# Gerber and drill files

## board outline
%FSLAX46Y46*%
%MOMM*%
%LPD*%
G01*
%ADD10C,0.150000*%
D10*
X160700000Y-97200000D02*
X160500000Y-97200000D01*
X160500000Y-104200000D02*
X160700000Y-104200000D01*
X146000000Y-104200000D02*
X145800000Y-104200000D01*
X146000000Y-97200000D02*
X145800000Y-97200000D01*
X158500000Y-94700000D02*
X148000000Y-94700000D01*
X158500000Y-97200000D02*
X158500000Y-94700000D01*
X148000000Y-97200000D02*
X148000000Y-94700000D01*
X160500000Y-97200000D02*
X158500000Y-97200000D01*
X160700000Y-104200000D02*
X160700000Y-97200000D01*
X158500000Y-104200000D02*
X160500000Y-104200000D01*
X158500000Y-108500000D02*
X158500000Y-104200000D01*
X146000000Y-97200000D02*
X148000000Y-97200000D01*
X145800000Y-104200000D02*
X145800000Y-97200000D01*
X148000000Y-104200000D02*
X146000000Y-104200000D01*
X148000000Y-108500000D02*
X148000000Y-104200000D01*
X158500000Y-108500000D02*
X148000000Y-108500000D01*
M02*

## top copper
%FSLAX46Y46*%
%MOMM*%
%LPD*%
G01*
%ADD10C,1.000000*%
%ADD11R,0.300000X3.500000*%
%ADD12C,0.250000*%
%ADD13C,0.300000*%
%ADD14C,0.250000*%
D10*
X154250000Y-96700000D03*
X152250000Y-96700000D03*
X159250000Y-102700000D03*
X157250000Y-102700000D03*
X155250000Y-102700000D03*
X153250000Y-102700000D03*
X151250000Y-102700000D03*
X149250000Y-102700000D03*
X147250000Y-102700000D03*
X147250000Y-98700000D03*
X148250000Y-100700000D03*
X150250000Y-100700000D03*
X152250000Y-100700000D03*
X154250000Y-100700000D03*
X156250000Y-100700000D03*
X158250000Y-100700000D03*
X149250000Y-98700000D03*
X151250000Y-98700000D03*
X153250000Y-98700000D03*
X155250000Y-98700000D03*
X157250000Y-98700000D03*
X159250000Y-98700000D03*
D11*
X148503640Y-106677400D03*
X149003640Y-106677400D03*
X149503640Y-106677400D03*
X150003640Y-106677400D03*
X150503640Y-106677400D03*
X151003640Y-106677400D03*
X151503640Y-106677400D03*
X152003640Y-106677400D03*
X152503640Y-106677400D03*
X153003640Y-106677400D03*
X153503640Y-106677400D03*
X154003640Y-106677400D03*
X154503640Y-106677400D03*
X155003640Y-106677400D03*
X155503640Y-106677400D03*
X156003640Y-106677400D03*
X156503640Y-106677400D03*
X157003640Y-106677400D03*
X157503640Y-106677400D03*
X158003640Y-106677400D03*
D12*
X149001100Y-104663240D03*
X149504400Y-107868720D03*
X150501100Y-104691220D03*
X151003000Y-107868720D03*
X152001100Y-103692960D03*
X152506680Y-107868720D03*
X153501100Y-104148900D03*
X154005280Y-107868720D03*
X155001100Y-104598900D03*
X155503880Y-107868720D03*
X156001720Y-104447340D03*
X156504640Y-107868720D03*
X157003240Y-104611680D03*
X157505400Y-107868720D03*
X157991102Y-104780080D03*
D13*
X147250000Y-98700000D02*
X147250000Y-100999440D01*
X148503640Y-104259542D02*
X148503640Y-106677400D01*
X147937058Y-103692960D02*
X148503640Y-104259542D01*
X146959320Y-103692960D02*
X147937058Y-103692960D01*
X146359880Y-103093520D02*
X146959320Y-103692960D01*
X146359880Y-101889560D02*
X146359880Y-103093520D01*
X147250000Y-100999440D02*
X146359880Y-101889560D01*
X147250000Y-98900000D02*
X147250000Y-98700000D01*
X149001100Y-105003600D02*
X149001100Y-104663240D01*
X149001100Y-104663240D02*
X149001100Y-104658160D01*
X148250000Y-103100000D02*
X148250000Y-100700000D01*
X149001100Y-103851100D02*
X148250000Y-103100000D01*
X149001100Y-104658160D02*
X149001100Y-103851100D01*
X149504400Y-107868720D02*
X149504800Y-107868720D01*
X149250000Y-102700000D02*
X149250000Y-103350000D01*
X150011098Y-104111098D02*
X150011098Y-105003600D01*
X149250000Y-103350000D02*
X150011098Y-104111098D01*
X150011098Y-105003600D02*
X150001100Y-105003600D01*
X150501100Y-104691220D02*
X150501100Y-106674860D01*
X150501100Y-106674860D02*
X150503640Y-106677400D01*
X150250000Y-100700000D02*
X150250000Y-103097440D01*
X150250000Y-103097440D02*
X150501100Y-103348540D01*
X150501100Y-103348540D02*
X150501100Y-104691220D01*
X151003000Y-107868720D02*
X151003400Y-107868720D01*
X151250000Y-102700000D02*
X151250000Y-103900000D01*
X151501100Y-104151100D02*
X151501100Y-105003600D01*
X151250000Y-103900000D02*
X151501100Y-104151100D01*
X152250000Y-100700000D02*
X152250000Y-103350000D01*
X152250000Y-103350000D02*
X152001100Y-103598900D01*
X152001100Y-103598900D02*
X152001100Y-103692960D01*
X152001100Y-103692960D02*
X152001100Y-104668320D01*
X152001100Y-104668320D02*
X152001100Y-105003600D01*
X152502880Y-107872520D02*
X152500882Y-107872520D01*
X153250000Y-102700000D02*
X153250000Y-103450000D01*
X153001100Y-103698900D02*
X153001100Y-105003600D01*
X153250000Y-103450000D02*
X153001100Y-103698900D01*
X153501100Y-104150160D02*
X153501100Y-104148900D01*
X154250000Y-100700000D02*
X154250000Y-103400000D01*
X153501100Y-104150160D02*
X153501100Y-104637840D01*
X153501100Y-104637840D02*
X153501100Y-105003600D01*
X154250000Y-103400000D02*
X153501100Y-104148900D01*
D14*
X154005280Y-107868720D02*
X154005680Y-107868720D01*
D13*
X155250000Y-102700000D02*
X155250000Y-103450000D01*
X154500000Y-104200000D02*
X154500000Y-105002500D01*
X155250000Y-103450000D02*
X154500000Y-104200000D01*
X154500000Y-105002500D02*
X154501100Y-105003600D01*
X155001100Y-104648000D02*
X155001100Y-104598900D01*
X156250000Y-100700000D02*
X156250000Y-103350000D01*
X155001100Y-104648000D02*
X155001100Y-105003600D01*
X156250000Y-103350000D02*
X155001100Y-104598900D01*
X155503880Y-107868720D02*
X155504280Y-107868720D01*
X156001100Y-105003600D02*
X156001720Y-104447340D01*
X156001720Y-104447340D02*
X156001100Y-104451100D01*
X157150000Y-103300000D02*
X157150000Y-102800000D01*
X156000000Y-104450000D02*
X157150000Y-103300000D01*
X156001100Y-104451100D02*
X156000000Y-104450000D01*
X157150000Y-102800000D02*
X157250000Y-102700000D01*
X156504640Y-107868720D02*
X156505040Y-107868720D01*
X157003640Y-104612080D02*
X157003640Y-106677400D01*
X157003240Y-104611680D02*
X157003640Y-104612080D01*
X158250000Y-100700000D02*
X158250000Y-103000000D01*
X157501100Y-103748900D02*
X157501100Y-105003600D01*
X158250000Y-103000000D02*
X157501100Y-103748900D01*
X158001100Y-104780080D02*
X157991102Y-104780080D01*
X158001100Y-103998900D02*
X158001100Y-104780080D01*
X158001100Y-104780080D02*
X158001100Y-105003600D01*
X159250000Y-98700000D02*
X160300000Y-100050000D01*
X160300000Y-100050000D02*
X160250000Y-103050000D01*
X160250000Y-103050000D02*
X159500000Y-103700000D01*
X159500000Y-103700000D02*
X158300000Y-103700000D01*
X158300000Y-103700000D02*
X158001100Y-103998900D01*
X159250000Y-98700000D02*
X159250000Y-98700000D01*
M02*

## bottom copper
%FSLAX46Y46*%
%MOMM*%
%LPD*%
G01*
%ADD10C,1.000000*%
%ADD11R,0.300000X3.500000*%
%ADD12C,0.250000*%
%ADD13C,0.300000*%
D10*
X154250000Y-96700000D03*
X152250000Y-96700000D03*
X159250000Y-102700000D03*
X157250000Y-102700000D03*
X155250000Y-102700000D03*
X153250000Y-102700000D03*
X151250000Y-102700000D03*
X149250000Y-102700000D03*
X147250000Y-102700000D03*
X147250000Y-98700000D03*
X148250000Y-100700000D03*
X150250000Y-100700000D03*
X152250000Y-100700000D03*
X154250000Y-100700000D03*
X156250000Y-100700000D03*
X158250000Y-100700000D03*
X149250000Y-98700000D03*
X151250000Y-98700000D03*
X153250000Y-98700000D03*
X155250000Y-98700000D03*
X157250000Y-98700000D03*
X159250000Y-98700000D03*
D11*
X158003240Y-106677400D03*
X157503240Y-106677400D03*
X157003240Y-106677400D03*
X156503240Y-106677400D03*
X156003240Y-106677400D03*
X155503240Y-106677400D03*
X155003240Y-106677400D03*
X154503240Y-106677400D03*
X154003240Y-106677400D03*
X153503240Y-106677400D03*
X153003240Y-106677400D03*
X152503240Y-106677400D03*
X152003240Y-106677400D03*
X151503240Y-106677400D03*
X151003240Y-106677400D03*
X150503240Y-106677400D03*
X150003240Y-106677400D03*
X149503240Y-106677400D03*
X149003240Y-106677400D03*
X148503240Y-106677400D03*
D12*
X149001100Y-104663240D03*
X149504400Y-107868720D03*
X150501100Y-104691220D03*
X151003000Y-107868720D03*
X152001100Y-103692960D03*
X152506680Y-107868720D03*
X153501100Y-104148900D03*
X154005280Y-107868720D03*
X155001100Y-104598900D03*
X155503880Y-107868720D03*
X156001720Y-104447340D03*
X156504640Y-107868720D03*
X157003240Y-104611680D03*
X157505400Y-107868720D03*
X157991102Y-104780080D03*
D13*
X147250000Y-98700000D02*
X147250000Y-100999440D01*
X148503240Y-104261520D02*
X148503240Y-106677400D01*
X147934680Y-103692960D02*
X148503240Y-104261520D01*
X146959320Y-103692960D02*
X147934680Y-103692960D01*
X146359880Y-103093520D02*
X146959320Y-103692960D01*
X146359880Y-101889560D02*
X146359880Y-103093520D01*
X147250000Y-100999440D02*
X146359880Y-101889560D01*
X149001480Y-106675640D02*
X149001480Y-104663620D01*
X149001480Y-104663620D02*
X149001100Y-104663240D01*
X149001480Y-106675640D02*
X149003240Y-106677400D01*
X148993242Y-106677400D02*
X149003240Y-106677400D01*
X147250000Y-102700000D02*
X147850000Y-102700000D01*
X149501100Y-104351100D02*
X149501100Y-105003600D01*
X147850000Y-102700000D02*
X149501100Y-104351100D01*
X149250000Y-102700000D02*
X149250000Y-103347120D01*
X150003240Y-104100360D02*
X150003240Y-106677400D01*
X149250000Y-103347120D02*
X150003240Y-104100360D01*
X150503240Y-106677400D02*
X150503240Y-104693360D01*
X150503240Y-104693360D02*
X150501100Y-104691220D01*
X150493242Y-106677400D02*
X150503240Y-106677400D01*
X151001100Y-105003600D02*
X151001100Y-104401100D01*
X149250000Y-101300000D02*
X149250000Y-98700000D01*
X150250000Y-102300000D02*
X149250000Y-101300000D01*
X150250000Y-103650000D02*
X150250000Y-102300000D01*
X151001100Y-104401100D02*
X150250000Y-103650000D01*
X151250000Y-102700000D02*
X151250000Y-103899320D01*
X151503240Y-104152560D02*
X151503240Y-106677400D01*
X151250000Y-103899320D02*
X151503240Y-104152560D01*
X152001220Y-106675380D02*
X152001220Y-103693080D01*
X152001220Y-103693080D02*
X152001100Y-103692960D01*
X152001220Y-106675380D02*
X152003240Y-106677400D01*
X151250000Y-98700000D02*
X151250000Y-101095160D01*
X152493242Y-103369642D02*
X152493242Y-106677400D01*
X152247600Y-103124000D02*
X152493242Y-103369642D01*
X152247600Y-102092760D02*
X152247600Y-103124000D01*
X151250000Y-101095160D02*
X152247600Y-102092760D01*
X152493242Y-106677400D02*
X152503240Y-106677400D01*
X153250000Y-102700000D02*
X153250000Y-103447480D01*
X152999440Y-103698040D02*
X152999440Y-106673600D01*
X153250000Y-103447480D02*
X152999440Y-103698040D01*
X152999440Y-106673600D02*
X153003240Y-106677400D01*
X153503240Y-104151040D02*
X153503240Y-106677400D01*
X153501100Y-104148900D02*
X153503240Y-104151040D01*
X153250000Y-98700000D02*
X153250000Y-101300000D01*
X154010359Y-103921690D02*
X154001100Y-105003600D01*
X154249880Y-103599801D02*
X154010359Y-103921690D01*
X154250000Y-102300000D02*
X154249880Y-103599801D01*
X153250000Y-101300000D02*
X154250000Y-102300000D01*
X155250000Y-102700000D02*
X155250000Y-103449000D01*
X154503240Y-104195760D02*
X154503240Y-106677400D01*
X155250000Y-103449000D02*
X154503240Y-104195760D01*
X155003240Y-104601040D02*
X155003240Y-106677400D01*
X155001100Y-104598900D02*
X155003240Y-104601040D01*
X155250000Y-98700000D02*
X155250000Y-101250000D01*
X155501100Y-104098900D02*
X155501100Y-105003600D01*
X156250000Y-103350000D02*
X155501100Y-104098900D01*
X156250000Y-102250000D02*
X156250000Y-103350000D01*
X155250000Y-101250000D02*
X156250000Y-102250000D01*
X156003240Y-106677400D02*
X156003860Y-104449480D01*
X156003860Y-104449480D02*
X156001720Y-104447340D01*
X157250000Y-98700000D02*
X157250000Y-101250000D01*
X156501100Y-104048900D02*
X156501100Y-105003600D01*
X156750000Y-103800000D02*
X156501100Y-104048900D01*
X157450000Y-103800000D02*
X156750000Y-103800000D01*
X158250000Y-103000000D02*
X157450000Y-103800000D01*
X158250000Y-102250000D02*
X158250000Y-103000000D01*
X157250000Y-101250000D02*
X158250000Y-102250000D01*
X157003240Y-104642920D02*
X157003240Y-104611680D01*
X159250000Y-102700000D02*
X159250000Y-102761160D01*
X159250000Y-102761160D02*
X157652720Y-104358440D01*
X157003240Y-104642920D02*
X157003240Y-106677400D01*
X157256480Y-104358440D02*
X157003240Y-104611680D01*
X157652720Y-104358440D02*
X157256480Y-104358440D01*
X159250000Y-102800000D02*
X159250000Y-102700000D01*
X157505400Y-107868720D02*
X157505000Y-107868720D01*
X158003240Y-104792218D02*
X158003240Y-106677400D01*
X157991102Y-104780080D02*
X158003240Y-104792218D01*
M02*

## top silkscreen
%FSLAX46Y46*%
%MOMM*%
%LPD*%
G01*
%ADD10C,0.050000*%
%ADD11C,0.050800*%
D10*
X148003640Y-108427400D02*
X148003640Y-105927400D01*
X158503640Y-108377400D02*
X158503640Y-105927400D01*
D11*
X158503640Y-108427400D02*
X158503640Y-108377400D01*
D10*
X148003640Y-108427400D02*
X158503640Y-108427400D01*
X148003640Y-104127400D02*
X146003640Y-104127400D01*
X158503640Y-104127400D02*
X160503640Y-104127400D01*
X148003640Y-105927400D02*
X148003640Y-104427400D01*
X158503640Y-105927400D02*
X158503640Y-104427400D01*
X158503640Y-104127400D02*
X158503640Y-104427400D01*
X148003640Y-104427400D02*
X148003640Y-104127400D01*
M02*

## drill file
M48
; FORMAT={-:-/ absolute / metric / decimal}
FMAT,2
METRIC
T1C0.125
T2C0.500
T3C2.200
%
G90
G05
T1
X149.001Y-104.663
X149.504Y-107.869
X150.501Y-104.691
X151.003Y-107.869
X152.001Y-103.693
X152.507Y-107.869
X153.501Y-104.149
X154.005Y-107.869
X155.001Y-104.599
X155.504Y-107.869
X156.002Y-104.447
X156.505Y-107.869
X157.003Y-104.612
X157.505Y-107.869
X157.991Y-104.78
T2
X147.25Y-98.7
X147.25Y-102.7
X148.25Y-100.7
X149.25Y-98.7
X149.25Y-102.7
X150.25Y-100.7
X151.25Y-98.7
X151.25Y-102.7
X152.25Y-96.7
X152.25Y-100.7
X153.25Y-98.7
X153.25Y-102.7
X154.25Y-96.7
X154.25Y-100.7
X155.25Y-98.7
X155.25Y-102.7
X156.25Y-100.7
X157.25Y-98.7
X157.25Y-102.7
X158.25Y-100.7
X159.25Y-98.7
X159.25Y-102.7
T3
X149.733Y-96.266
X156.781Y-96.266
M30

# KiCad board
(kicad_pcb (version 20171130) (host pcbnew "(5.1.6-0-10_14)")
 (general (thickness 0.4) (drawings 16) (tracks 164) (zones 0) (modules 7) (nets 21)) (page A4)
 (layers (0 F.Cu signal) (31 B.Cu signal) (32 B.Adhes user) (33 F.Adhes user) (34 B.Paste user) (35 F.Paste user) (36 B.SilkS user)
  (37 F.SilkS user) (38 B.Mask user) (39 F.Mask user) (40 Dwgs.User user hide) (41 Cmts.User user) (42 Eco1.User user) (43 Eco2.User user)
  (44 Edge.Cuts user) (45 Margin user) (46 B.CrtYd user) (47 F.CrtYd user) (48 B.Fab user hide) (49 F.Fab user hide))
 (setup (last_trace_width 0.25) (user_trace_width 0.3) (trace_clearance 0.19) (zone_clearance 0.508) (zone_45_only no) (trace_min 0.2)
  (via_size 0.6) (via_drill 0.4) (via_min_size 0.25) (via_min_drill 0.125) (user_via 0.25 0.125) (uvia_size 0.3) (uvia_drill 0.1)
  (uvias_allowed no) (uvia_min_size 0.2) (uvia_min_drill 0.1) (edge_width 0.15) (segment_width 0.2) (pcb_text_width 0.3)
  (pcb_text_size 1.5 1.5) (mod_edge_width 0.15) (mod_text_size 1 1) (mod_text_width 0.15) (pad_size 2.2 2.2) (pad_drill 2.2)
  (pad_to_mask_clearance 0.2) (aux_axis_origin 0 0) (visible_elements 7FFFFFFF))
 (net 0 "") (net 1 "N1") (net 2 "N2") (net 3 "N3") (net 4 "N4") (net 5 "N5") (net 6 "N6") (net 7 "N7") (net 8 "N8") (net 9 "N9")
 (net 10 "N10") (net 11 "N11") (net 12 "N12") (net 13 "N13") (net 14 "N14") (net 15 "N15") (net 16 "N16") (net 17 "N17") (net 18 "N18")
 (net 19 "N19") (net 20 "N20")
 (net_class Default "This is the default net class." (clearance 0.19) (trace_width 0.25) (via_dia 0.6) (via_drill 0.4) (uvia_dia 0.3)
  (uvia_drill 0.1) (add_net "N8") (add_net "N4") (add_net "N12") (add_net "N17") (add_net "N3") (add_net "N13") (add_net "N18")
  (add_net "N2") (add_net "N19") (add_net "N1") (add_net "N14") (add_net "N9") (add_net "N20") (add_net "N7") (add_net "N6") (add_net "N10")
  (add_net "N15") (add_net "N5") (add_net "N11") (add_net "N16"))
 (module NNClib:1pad (layer F.Cu) (at 154.25 96.7)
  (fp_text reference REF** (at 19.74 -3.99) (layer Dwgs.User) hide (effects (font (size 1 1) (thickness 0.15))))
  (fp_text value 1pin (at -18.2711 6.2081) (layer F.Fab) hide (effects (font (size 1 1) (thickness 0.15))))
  (pad 1 thru_hole circle (at 0 0) (size 1 1) (drill 0.5) (layers *.Cu *.Mask)))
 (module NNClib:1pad (layer F.Cu) (at 152.25 96.7)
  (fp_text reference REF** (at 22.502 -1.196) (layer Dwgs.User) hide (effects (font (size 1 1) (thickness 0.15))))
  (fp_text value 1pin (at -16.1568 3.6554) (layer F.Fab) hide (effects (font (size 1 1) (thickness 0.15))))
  (pad 1 thru_hole circle (at 0 0) (size 1 1) (drill 0.5) (layers *.Cu *.Mask)))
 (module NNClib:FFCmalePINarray (layer F.Cu) (at 147.25 102.7)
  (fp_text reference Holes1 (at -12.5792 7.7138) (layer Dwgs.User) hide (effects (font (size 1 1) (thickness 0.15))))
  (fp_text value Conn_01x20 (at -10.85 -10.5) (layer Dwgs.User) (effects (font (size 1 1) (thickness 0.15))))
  (pad 18 thru_hole circle (at 12 0) (size 1 1) (drill 0.5) (layers *.Cu *.Mask) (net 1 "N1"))
  (pad 16 thru_hole circle (at 10 0) (size 1 1) (drill 0.5) (layers *.Cu *.Mask) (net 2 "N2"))
  (pad 13 thru_hole circle (at 8 0) (size 1 1) (drill 0.5) (layers *.Cu *.Mask) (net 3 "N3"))
  (pad 10 thru_hole circle (at 6 0) (size 1 1) (drill 0.5) (layers *.Cu *.Mask) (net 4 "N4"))
  (pad 7 thru_hole circle (at 4 0) (size 1 1) (drill 0.5) (layers *.Cu *.Mask) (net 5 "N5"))
  (pad 4 thru_hole circle (at 2 0) (size 1 1) (drill 0.5) (layers *.Cu *.Mask) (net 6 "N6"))
  (pad 3 thru_hole circle (at 0 0) (size 1 1) (drill 0.5) (layers *.Cu *.Mask) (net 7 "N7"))
  (pad 1 thru_hole circle (at 0 -4) (size 1 1) (drill 0.5) (layers *.Cu *.Mask) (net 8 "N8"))
  (pad 2 thru_hole circle (at 1 -2) (size 1 1) (drill 0.5) (layers *.Cu *.Mask) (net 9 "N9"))
  (pad 5 thru_hole circle (at 3 -2) (size 1 1) (drill 0.5) (layers *.Cu *.Mask) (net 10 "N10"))
  (pad 8 thru_hole circle (at 5 -2) (size 1 1) (drill 0.5) (layers *.Cu *.Mask) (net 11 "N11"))
  (pad 11 thru_hole circle (at 7 -2) (size 1 1) (drill 0.5) (layers *.Cu *.Mask) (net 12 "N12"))
  (pad 14 thru_hole circle (at 9 -2) (size 1 1) (drill 0.5) (layers *.Cu *.Mask) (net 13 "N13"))
  (pad 19 thru_hole circle (at 11 -2) (size 1 1) (drill 0.5) (layers *.Cu *.Mask) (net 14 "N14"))
  (pad 6 thru_hole circle (at 2 -4) (size 1 1) (drill 0.5) (layers *.Cu *.Mask) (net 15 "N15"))
  (pad 9 thru_hole circle (at 4 -4) (size 1 1) (drill 0.5) (layers *.Cu *.Mask) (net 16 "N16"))
  (pad 12 thru_hole circle (at 6 -4) (size 1 1) (drill 0.5) (layers *.Cu *.Mask) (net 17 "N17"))
  (pad 15 thru_hole circle (at 8 -4) (size 1 1) (drill 0.5) (layers *.Cu *.Mask) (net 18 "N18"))
  (pad 17 thru_hole circle (at 10 -4) (size 1 1) (drill 0.5) (layers *.Cu *.Mask) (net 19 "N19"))
  (pad 20 thru_hole circle (at 12 -4) (size 1 1) (drill 0.5) (layers *.Cu *.Mask) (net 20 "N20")))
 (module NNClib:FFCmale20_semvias (layer F.Cu) (at 148.50364 104.9274)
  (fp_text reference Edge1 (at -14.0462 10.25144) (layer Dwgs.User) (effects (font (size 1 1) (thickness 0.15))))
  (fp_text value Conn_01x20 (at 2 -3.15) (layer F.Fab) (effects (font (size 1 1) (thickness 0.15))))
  (fp_line (start -0.5 3.5) (end -0.5 1) (layer F.SilkS) (width 0.05))
  (fp_line (start 10 3.45) (end 10 1) (layer F.SilkS) (width 0.05))
  (fp_line (start 10 3.5) (end 10 3.45) (layer F.SilkS) (width 0.0508))
  (fp_line (start -0.5 3.5) (end 10 3.5) (layer F.SilkS) (width 0.05))
  (fp_line (start -0.5 -0.8) (end -2.5 -0.8) (layer F.SilkS) (width 0.05))
  (fp_line (start 10 -0.8) (end 12 -0.8) (layer F.SilkS) (width 0.05))
  (fp_line (start -0.5 1) (end -0.5 -0.5) (layer F.SilkS) (width 0.05))
  (fp_line (start 10 1) (end 10 -0.5) (layer F.SilkS) (width 0.05))
  (fp_line (start 10 -0.8) (end 10 -0.5) (layer F.SilkS) (width 0.05))
  (fp_line (start -0.5 -0.5) (end -0.5 -0.8) (layer F.SilkS) (width 0.05))
  (pad 1 smd rect (at 0 1.75) (size 0.3 3.5) (layers *.Paste *.Mask F.Cu) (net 8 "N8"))
  (pad 2 smd rect (at 0.5 1.75) (size 0.3 3.5) (layers *.Paste *.Mask F.Cu) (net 9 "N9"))
  (pad 3 smd rect (at 1 1.75) (size 0.3 3.5) (layers *.Paste *.Mask F.Cu) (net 7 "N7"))
  (pad 4 smd rect (at 1.5 1.75) (size 0.3 3.5) (layers *.Paste *.Mask F.Cu) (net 6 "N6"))
  (pad 5 smd rect (at 2 1.75) (size 0.3 3.5) (layers *.Paste *.Mask F.Cu) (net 10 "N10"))
  (pad 6 smd rect (at 2.5 1.75) (size 0.3 3.5) (layers *.Paste *.Mask F.Cu) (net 15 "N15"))
  (pad 7 smd rect (at 3 1.75) (size 0.3 3.5) (layers *.Paste *.Mask F.Cu) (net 5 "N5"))
  (pad 8 smd rect (at 3.5 1.75) (size 0.3 3.5) (layers *.Paste *.Mask F.Cu) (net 11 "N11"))
  (pad 9 smd rect (at 4 1.75) (size 0.3 3.5) (layers *.Paste *.Mask F.Cu) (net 16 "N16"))
  (pad 10 smd rect (at 4.5 1.75) (size 0.3 3.5) (layers *.Paste *.Mask F.Cu) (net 4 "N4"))
  (pad 11 smd rect (at 5 1.75) (size 0.3 3.5) (layers *.Paste *.Mask F.Cu) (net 12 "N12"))
  (pad 12 smd rect (at 5.5 1.75) (size 0.3 3.5) (layers *.Paste *.Mask F.Cu) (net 17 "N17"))
  (pad 13 smd rect (at 6 1.75) (size 0.3 3.5) (layers *.Paste *.Mask F.Cu) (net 3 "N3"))
  (pad 14 smd rect (at 6.5 1.75) (size 0.3 3.5) (layers *.Paste *.Mask F.Cu) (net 13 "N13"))
  (pad 15 smd rect (at 7 1.75) (size 0.3 3.5) (layers *.Paste *.Mask F.Cu) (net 18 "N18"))
  (pad 16 smd rect (at 7.5 1.75) (size 0.3 3.5) (layers *.Paste *.Mask F.Cu) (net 2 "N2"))
  (pad 17 smd rect (at 8 1.75) (size 0.3 3.5) (layers *.Paste *.Mask F.Cu) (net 19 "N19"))
  (pad 18 smd rect (at 8.5 1.75) (size 0.3 3.5) (layers *.Paste *.Mask F.Cu) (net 1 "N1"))
  (pad 19 smd rect (at 9 1.75) (size 0.3 3.5) (layers *.Paste *.Mask F.Cu) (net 14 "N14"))
  (pad 20 smd rect (at 9.5 1.75) (size 0.3 3.5) (layers *.Paste *.Mask F.Cu) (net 20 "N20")))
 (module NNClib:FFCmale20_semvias (layer B.Cu) (at 158.00324 104.9274 180)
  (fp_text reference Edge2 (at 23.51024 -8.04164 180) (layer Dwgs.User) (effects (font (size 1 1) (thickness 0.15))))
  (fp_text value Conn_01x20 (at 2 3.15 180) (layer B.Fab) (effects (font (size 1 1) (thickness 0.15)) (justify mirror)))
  (pad 1 smd rect (at 0 -1.75 180) (size 0.3 3.5) (layers *.Paste *.Mask B.Cu) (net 20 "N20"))
  (pad 2 smd rect (at 0.5 -1.75 180) (size 0.3 3.5) (layers *.Paste *.Mask B.Cu) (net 14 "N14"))
  (pad 3 smd rect (at 1 -1.75 180) (size 0.3 3.5) (layers *.Paste *.Mask B.Cu) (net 1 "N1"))
  (pad 4 smd rect (at 1.5 -1.75 180) (size 0.3 3.5) (layers *.Paste *.Mask B.Cu) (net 19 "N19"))
  (pad 5 smd rect (at 2 -1.75 180) (size 0.3 3.5) (layers *.Paste *.Mask B.Cu) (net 2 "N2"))
  (pad 6 smd rect (at 2.5 -1.75 180) (size 0.3 3.5) (layers *.Paste *.Mask B.Cu) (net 18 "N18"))
  (pad 7 smd rect (at 3 -1.75 180) (size 0.3 3.5) (layers *.Paste *.Mask B.Cu) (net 13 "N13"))
  (pad 8 smd rect (at 3.5 -1.75 180) (size 0.3 3.5) (layers *.Paste *.Mask B.Cu) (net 3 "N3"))
  (pad 9 smd rect (at 4 -1.75 180) (size 0.3 3.5) (layers *.Paste *.Mask B.Cu) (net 17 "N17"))
  (pad 10 smd rect (at 4.5 -1.75 180) (size 0.3 3.5) (layers *.Paste *.Mask B.Cu) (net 12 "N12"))
  (pad 11 smd rect (at 5 -1.75 180) (size 0.3 3.5) (layers *.Paste *.Mask B.Cu) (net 4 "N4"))
  (pad 12 smd rect (at 5.5 -1.75 180) (size 0.3 3.5) (layers *.Paste *.Mask B.Cu) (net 16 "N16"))
  (pad 13 smd rect (at 6 -1.75 180) (size 0.3 3.5) (layers *.Paste *.Mask B.Cu) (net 11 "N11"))
  (pad 14 smd rect (at 6.5 -1.75 180) (size 0.3 3.5) (layers *.Paste *.Mask B.Cu) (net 5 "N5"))
  (pad 15 smd rect (at 7 -1.75 180) (size 0.3 3.5) (layers *.Paste *.Mask B.Cu) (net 15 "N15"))
  (pad 16 smd rect (at 7.5 -1.75 180) (size 0.3 3.5) (layers *.Paste *.Mask B.Cu) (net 10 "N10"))
  (pad 17 smd rect (at 8 -1.75 180) (size 0.3 3.5) (layers *.Paste *.Mask B.Cu) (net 6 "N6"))
  (pad 18 smd rect (at 8.5 -1.75 180) (size 0.3 3.5) (layers *.Paste *.Mask B.Cu) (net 7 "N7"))
  (pad 19 smd rect (at 9 -1.75 180) (size 0.3 3.5) (layers *.Paste *.Mask B.Cu) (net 9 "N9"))
  (pad 20 smd rect (at 9.5 -1.75 180) (size 0.3 3.5) (layers *.Paste *.Mask B.Cu) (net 8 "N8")))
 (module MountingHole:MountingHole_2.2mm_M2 (layer F.Cu) (at 149.733 96.266)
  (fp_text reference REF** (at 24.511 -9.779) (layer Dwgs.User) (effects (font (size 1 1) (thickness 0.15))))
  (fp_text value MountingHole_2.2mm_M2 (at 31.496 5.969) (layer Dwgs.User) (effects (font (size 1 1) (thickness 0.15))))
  (pad 1 np_thru_hole circle (at 0 0) (size 2.2 2.2) (drill 2.2) (layers *.Cu *.Mask)))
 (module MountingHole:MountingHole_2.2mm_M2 (layer F.Cu) (at 156.7815 96.266)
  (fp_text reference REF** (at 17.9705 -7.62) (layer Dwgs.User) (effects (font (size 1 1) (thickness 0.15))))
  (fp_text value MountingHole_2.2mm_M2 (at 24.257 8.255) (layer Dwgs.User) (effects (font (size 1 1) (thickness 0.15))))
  (pad 1 np_thru_hole circle (at 0 0) (size 2.2 2.2) (drill 2.2) (layers *.Cu *.Mask)))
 (gr_line (start 160.7 97.2) (end 160.5 97.2) (angle 90) (layer Edge.Cuts) (width 0.15))
 (gr_line (start 160.5 104.2) (end 160.7 104.2) (angle 90) (layer Edge.Cuts) (width 0.15))
 (gr_line (start 146 104.2) (end 145.8 104.2) (angle 90) (layer Edge.Cuts) (width 0.15))
 (gr_line (start 146 97.2) (end 145.8 97.2) (angle 90) (layer Edge.Cuts) (width 0.15))
 (gr_line (start 158.5 94.7) (end 148 94.7) (angle 90) (layer Edge.Cuts) (width 0.15))
 (gr_line (start 158.5 97.2) (end 158.5 94.7) (angle 90) (layer Edge.Cuts) (width 0.15))
 (gr_line (start 148 97.2) (end 148 94.7) (angle 90) (layer Edge.Cuts) (width 0.15))
 (gr_line (start 160.5 97.2) (end 158.5 97.2) (angle 90) (layer Edge.Cuts) (width 0.15))
 (gr_line (start 160.7 104.2) (end 160.7 97.2) (angle 90) (layer Edge.Cuts) (width 0.15))
 (gr_line (start 158.5 104.2) (end 160.5 104.2) (angle 90) (layer Edge.Cuts) (width 0.15))
 (gr_line (start 158.5 108.5) (end 158.5 104.2) (angle 90) (layer Edge.Cuts) (width 0.15))
 (gr_line (start 146 97.2) (end 148 97.2) (angle 90) (layer Edge.Cuts) (width 0.15))
 (gr_line (start 145.8 104.2) (end 145.8 97.2) (angle 90) (layer Edge.Cuts) (width 0.15))
 (gr_line (start 148 104.2) (end 146 104.2) (angle 90) (layer Edge.Cuts) (width 0.15))
 (gr_line (start 148 108.5) (end 148 104.2) (angle 90) (layer Edge.Cuts) (width 0.15))
 (gr_line (start 158.5 108.5) (end 148 108.5) (angle 90) (layer Edge.Cuts) (width 0.15))
 (segment (start 147.25 98.7) (end 147.25 100.99944) (width 0.3) (layer B.Cu) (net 8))
 (segment (start 148.50324 104.26152) (end 148.50324 106.6774) (width 0.3) (layer B.Cu) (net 8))
 (segment (start 147.93468 103.69296) (end 148.50324 104.26152) (width 0.3) (layer B.Cu) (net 8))
 (segment (start 146.95932 103.69296) (end 147.93468 103.69296) (width 0.3) (layer B.Cu) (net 8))
 (segment (start 146.35988 103.09352) (end 146.95932 103.69296) (width 0.3) (layer B.Cu) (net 8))
 (segment (start 146.35988 101.88956) (end 146.35988 103.09352) (width 0.3) (layer B.Cu) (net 8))
 (segment (start 147.25 100.99944) (end 146.35988 101.88956) (width 0.3) (layer B.Cu) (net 8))
 (segment (start 147.25 98.7) (end 147.25 100.99944) (width 0.3) (layer F.Cu) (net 8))
 (segment (start 148.50364 104.259542) (end 148.50364 106.6774) (width 0.3) (layer F.Cu) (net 8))
 (segment (start 147.937058 103.69296) (end 148.50364 104.259542) (width 0.3) (layer F.Cu) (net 8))
 (segment (start 146.95932 103.69296) (end 147.937058 103.69296) (width 0.3) (layer F.Cu) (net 8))
 (segment (start 146.35988 103.09352) (end 146.95932 103.69296) (width 0.3) (layer F.Cu) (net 8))
 (segment (start 146.35988 101.88956) (end 146.35988 103.09352) (width 0.3) (layer F.Cu) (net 8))
 (segment (start 147.25 100.99944) (end 146.35988 101.88956) (width 0.3) (layer F.Cu) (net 8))
 (segment (start 147.25 98.9) (end 147.25 98.7) (width 0.3) (layer F.Cu) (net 8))
 (via (at 149.0011 104.66324) (size 0.25) (drill 0.125) (layers F.Cu B.Cu) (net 9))
 (segment (start 149.00148 106.67564) (end 149.00148 104.66362) (width 0.3) (layer B.Cu) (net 9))
 (segment (start 149.00148 104.66362) (end 149.0011 104.66324) (width 0.3) (layer B.Cu) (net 9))
 (segment (start 149.00148 106.67564) (end 149.00324 106.6774) (width 0.3) (layer B.Cu) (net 9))
 (segment (start 148.993242 106.6774) (end 149.00324 106.6774) (width 0.3) (layer B.Cu) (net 9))
 (segment (start 149.0011 105.0036) (end 149.0011 104.66324) (width 0.3) (layer F.Cu) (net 9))
 (segment (start 149.0011 104.66324) (end 149.0011 104.65816) (width 0.3) (layer F.Cu) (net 9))
 (segment (start 148.25 103.1) (end 148.25 100.7) (width 0.3) (layer F.Cu) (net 9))
 (segment (start 149.0011 103.8511) (end 148.25 103.1) (width 0.3) (layer F.Cu) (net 9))
 (segment (start 149.0011 104.65816) (end 149.0011 103.8511) (width 0.3) (layer F.Cu) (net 9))
 (segment (start 149.5044 107.86872) (end 149.5048 107.86872) (width 0.3) (layer F.Cu) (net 7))
 (via (at 149.5044 107.86872) (size 0.25) (drill 0.125) (layers F.Cu B.Cu) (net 7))
 (segment (start 147.25 102.7) (end 147.85 102.7) (width 0.3) (layer B.Cu) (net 7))
 (segment (start 149.5011 104.3511) (end 149.5011 105.0036) (width 0.3) (layer B.Cu) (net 7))
 (segment (start 147.85 102.7) (end 149.5011 104.3511) (width 0.3) (layer B.Cu) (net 7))
 (segment (start 149.25 102.7) (end 149.25 103.34712) (width 0.3) (layer B.Cu) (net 6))
 (segment (start 150.00324 104.10036) (end 150.00324 106.6774) (width 0.3) (layer B.Cu) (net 6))
 (segment (start 149.25 103.34712) (end 150.00324 104.10036) (width 0.3) (layer B.Cu) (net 6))
 (segment (start 149.25 102.7) (end 149.25 103.35) (width 0.3) (layer F.Cu) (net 6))
 (segment (start 150.011098 104.111098) (end 150.011098 105.0036) (width 0.3) (layer F.Cu) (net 6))
 (segment (start 149.25 103.35) (end 150.011098 104.111098) (width 0.3) (layer F.Cu) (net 6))
 (segment (start 150.011098 105.0036) (end 150.0011 105.0036) (width 0.3) (layer F.Cu) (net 6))
 (via (at 150.5011 104.69122) (size 0.25) (drill 0.125) (layers F.Cu B.Cu) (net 10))
 (segment (start 150.50324 106.6774) (end 150.50324 104.69336) (width 0.3) (layer B.Cu) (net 10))
 (segment (start 150.50324 104.69336) (end 150.5011 104.69122) (width 0.3) (layer B.Cu) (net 10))
 (segment (start 150.5011 104.69122) (end 150.5011 106.67486) (width 0.3) (layer F.Cu) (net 10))
 (segment (start 150.5011 106.67486) (end 150.50364 106.6774) (width 0.3) (layer F.Cu) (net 10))
 (segment (start 150.25 100.7) (end 150.25 103.09744) (width 0.3) (layer F.Cu) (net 10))
 (segment (start 150.25 103.09744) (end 150.5011 103.34854) (width 0.3) (layer F.Cu) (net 10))
 (segment (start 150.5011 103.34854) (end 150.5011 104.69122) (width 0.3) (layer F.Cu) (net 10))
 (segment (start 150.493242 106.6774) (end 150.50324 106.6774) (width 0.3) (layer B.Cu) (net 10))
 (segment (start 151.003 107.86872) (end 151.0034 107.86872) (width 0.3) (layer F.Cu) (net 15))
 (via (at 151.003 107.86872) (size 0.25) (drill 0.125) (layers F.Cu B.Cu) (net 15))
 (segment (start 151.0011 105.0036) (end 151.0011 104.4011) (width 0.3) (layer B.Cu) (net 15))
 (segment (start 149.25 101.3) (end 149.25 98.7) (width 0.3) (layer B.Cu) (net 15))
 (segment (start 150.25 102.3) (end 149.25 101.3) (width 0.3) (layer B.Cu) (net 15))
 (segment (start 150.25 103.65) (end 150.25 102.3) (width 0.3) (layer B.Cu) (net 15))
 (segment (start 151.0011 104.4011) (end 150.25 103.65) (width 0.3) (layer B.Cu) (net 15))
 (segment (start 151.25 102.7) (end 151.25 103.89932) (width 0.3) (layer B.Cu) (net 5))
 (segment (start 151.50324 104.15256) (end 151.50324 106.6774) (width 0.3) (layer B.Cu) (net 5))
 (segment (start 151.25 103.89932) (end 151.50324 104.15256) (width 0.3) (layer B.Cu) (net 5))
 (segment (start 151.25 102.7) (end 151.25 103.9) (width 0.3) (layer F.Cu) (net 5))
 (segment (start 151.5011 104.1511) (end 151.5011 105.0036) (width 0.3) (layer F.Cu) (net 5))
 (segment (start 151.25 103.9) (end 151.5011 104.1511) (width 0.3) (layer F.Cu) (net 5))
 (via (at 152.0011 103.69296) (size 0.25) (drill 0.125) (layers F.Cu B.Cu) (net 11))
 (segment (start 152.00122 106.67538) (end 152.00122 103.69308) (width 0.3) (layer B.Cu) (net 11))
 (segment (start 152.00122 103.69308) (end 152.0011 103.69296) (width 0.3) (layer B.Cu) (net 11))
 (segment (start 152.00122 106.67538) (end 152.00324 106.6774) (width 0.3) (layer B.Cu) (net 11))
 (segment (start 152.25 100.7) (end 152.25 103.35) (width 0.3) (layer F.Cu) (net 11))
 (segment (start 152.25 103.35) (end 152.0011 103.5989) (width 0.3) (layer F.Cu) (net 11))
 (segment (start 152.0011 103.5989) (end 152.0011 103.69296) (width 0.3) (layer F.Cu) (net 11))
 (segment (start 152.0011 103.69296) (end 152.0011 104.66832) (width 0.3) (layer F.Cu) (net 11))
 (segment (start 152.0011 104.66832) (end 152.0011 105.0036) (width 0.3) (layer F.Cu) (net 11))
 (segment (start 151.25 98.7) (end 151.25 101.09516) (width 0.3) (layer B.Cu) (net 16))
 (segment (start 152.493242 103.369642) (end 152.493242 106.6774) (width 0.3) (layer B.Cu) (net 16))
 (segment (start 152.2476 103.124) (end 152.493242 103.369642) (width 0.3) (layer B.Cu) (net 16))
 (segment (start 152.2476 102.09276) (end 152.2476 103.124) (width 0.3) (layer B.Cu) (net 16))
 (segment (start 151.25 101.09516) (end 152.2476 102.09276) (width 0.3) (layer B.Cu) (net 16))
 (segment (start 152.493242 106.6774) (end 152.50324 106.6774) (width 0.3) (layer B.Cu) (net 16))
 (via (at 152.50668 107.86872) (size 0.25) (drill 0.125) (layers F.Cu B.Cu) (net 16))
 (segment (start 152.50288 107.87252) (end 152.500882 107.87252) (width 0.3) (layer F.Cu) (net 16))
 (segment (start 153.25 102.7) (end 153.25 103.44748) (width 0.3) (layer B.Cu) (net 4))
 (segment (start 152.99944 103.69804) (end 152.99944 106.6736) (width 0.3) (layer B.Cu) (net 4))
 (segment (start 153.25 103.44748) (end 152.99944 103.69804) (width 0.3) (layer B.Cu) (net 4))
 (segment (start 152.99944 106.6736) (end 153.00324 106.6774) (width 0.3) (layer B.Cu) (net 4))
 (segment (start 153.25 102.7) (end 153.25 103.45) (width 0.3) (layer F.Cu) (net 4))
 (segment (start 153.0011 103.6989) (end 153.0011 105.0036) (width 0.3) (layer F.Cu) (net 4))
 (segment (start 153.25 103.45) (end 153.0011 103.6989) (width 0.3) (layer F.Cu) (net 4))
 (segment (start 153.5011 104.15016) (end 153.5011 104.1489) (width 0.3) (layer F.Cu) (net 12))
 (via (at 153.5011 104.1489) (size 0.25) (drill 0.125) (layers F.Cu B.Cu) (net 12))
 (segment (start 153.50324 104.15104) (end 153.50324 106.6774) (width 0.3) (layer B.Cu) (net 12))
 (segment (start 153.5011 104.1489) (end 153.50324 104.15104) (width 0.3) (layer B.Cu) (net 12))
 (segment (start 154.25 100.7) (end 154.25 103.4) (width 0.3) (layer F.Cu) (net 12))
 (segment (start 153.5011 104.15016) (end 153.5011 104.63784) (width 0.3) (layer F.Cu) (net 12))
 (segment (start 153.5011 104.63784) (end 153.5011 105.0036) (width 0.3) (layer F.Cu) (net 12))
 (segment (start 154.25 103.4) (end 153.5011 104.1489) (width 0.3) (layer F.Cu) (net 12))
 (via (at 154.00528 107.86872) (size 0.25) (drill 0.125) (layers F.Cu B.Cu) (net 17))
 (segment (start 154.00528 107.86872) (end 154.00568 107.86872) (width 0.25) (layer F.Cu) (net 17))
 (segment (start 153.25 98.7) (end 153.25 101.3) (width 0.3) (layer B.Cu) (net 17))
 (segment (start 154.010359 103.92169) (end 154.0011 105.0036) (width 0.3) (layer B.Cu) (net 17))
 (segment (start 154.24988 103.599801) (end 154.010359 103.92169) (width 0.3) (layer B.Cu) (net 17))
 (segment (start 154.25 102.3) (end 154.24988 103.599801) (width 0.3) (layer B.Cu) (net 17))
 (segment (start 153.25 101.3) (end 154.25 102.3) (width 0.3) (layer B.Cu) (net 17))
 (segment (start 155.25 102.7) (end 155.25 103.449) (width 0.3) (layer B.Cu) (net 3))
 (segment (start 154.50324 104.19576) (end 154.50324 106.6774) (width 0.3) (layer B.Cu) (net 3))
 (segment (start 155.25 103.449) (end 154.50324 104.19576) (width 0.3) (layer B.Cu) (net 3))
 (segment (start 155.25 102.7) (end 155.25 103.45) (width 0.3) (layer F.Cu) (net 3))
 (segment (start 154.5 104.2) (end 154.5 105.0025) (width 0.3) (layer F.Cu) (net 3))
 (segment (start 155.25 103.45) (end 154.5 104.2) (width 0.3) (layer F.Cu) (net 3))
 (segment (start 154.5 105.0025) (end 154.5011 105.0036) (width 0.3) (layer F.Cu) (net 3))
 (segment (start 155.0011 104.648) (end 155.0011 104.5989) (width 0.3) (layer F.Cu) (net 13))
 (via (at 155.0011 104.5989) (size 0.25) (drill 0.125) (layers F.Cu B.Cu) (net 13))
 (segment (start 155.00324 104.60104) (end 155.00324 106.6774) (width 0.3) (layer B.Cu) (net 13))
 (segment (start 155.0011 104.5989) (end 155.00324 104.60104) (width 0.3) (layer B.Cu) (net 13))
 (segment (start 156.25 100.7) (end 156.25 103.35) (width 0.3) (layer F.Cu) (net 13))
 (segment (start 155.0011 104.648) (end 155.0011 105.0036) (width 0.3) (layer F.Cu) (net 13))
 (segment (start 156.25 103.35) (end 155.0011 104.5989) (width 0.3) (layer F.Cu) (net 13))
 (via (at 155.50388 107.86872) (size 0.25) (drill 0.125) (layers F.Cu B.Cu) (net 18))
 (segment (start 155.50388 107.86872) (end 155.50428 107.86872) (width 0.3) (layer F.Cu) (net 18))
 (segment (start 155.25 98.7) (end 155.25 101.25) (width 0.3) (layer B.Cu) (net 18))
 (segment (start 155.5011 104.0989) (end 155.5011 105.0036) (width 0.3) (layer B.Cu) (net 18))
 (segment (start 156.25 103.35) (end 155.5011 104.0989) (width 0.3) (layer B.Cu) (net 18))
 (segment (start 156.25 102.25) (end 156.25 103.35) (width 0.3) (layer B.Cu) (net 18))
 (segment (start 155.25 101.25) (end 156.25 102.25) (width 0.3) (layer B.Cu) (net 18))
 (via (at 156.00172 104.44734) (size 0.25) (drill 0.125) (layers F.Cu B.Cu) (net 2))
 (segment (start 156.00324 106.6774) (end 156.00386 104.44948) (width 0.3) (layer B.Cu) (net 2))
 (segment (start 156.00386 104.44948) (end 156.00172 104.44734) (width 0.3) (layer B.Cu) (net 2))
 (segment (start 156.0011 105.0036) (end 156.00172 104.44734) (width 0.3) (layer F.Cu) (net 2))
 (segment (start 156.00172 104.44734) (end 156.0011 104.4511) (width 0.3) (layer F.Cu) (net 2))
 (segment (start 157.15 103.3) (end 157.15 102.8) (width 0.3) (layer F.Cu) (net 2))
 (segment (start 156 104.45) (end 157.15 103.3) (width 0.3) (layer F.Cu) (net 2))
 (segment (start 156.0011 104.4511) (end 156 104.45) (width 0.3) (layer F.Cu) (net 2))
 (segment (start 157.15 102.8) (end 157.25 102.7) (width 0.3) (layer F.Cu) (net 2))
 (via (at 156.50464 107.86872) (size 0.25) (drill 0.125) (layers F.Cu B.Cu) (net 19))
 (segment (start 156.50464 107.86872) (end 156.50504 107.86872) (width 0.3) (layer F.Cu) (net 19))
 (segment (start 157.25 98.7) (end 157.25 101.25) (width 0.3) (layer B.Cu) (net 19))
 (segment (start 156.5011 104.0489) (end 156.5011 105.0036) (width 0.3) (layer B.Cu) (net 19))
 (segment (start 156.75 103.8) (end 156.5011 104.0489) (width 0.3) (layer B.Cu) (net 19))
 (segment (start 157.45 103.8) (end 156.75 103.8) (width 0.3) (layer B.Cu) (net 19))
 (segment (start 158.25 103) (end 157.45 103.8) (width 0.3) (layer B.Cu) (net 19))
 (segment (start 158.25 102.25) (end 158.25 103) (width 0.3) (layer B.Cu) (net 19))
 (segment (start 157.25 101.25) (end 158.25 102.25) (width 0.3) (layer B.Cu) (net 19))
 (segment (start 157.00324 104.64292) (end 157.00324 104.61168) (width 0.3) (layer B.Cu) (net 1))
 (via (at 157.00324 104.61168) (size 0.25) (drill 0.125) (layers F.Cu B.Cu) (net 1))
 (segment (start 157.00364 104.61208) (end 157.00364 106.6774) (width 0.3) (layer F.Cu) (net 1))
 (segment (start 157.00324 104.61168) (end 157.00364 104.61208) (width 0.3) (layer F.Cu) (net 1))
 (segment (start 159.25 102.7) (end 159.25 102.76116) (width 0.3) (layer B.Cu) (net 1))
 (segment (start 159.25 102.76116) (end 157.65272 104.35844) (width 0.3) (layer B.Cu) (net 1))
 (segment (start 157.00324 104.64292) (end 157.00324 106.6774) (width 0.3) (layer B.Cu) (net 1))
 (segment (start 157.25648 104.35844) (end 157.00324 104.61168) (width 0.3) (layer B.Cu) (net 1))
 (segment (start 157.65272 104.35844) (end 157.25648 104.35844) (width 0.3) (layer B.Cu) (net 1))
 (segment (start 159.25 102.8) (end 159.25 102.7) (width 0.3) (layer B.Cu) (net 1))
 (via (at 157.5054 107.86872) (size 0.25) (drill 0.125) (layers F.Cu B.Cu) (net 14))
 (segment (start 157.5054 107.86872) (end 157.505 107.86872) (width 0.3) (layer B.Cu) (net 14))
 (segment (start 158.25 100.7) (end 158.25 103) (width 0.3) (layer F.Cu) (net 14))
 (segment (start 157.5011 103.7489) (end 157.5011 105.0036) (width 0.3) (layer F.Cu) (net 14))
 (segment (start 158.25 103) (end 157.5011 103.7489) (width 0.3) (layer F.Cu) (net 14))
 (segment (start 158.0011 104.78008) (end 157.991102 104.78008) (width 0.3) (layer F.Cu) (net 20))
 (segment (start 158.00324 104.792218) (end 158.00324 106.6774) (width 0.3) (layer B.Cu) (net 20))
 (segment (start 157.991102 104.78008) (end 158.00324 104.792218) (width 0.3) (layer B.Cu) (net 20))
 (via (at 157.991102 104.78008) (size 0.25) (drill 0.125) (layers F.Cu B.Cu) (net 20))
 (segment (start 158.0011 103.9989) (end 158.0011 104.78008) (width 0.3) (layer F.Cu) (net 20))
 (segment (start 158.0011 104.78008) (end 158.0011 105.0036) (width 0.3) (layer F.Cu) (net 20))
 (segment (start 159.25 98.7) (end 160.3 100.05) (width 0.3) (layer F.Cu) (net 20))
 (segment (start 160.3 100.05) (end 160.25 103.05) (width 0.3) (layer F.Cu) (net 20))
 (segment (start 160.25 103.05) (end 159.5 103.7) (width 0.3) (layer F.Cu) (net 20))
 (segment (start 159.5 103.7) (end 158.3 103.7) (width 0.3) (layer F.Cu) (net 20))
 (segment (start 158.3 103.7) (end 158.0011 103.9989) (width 0.3) (layer F.Cu) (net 20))
 (segment (start 159.25 98.7) (end 159.25 98.7) (width 0.3) (layer F.Cu) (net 20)))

